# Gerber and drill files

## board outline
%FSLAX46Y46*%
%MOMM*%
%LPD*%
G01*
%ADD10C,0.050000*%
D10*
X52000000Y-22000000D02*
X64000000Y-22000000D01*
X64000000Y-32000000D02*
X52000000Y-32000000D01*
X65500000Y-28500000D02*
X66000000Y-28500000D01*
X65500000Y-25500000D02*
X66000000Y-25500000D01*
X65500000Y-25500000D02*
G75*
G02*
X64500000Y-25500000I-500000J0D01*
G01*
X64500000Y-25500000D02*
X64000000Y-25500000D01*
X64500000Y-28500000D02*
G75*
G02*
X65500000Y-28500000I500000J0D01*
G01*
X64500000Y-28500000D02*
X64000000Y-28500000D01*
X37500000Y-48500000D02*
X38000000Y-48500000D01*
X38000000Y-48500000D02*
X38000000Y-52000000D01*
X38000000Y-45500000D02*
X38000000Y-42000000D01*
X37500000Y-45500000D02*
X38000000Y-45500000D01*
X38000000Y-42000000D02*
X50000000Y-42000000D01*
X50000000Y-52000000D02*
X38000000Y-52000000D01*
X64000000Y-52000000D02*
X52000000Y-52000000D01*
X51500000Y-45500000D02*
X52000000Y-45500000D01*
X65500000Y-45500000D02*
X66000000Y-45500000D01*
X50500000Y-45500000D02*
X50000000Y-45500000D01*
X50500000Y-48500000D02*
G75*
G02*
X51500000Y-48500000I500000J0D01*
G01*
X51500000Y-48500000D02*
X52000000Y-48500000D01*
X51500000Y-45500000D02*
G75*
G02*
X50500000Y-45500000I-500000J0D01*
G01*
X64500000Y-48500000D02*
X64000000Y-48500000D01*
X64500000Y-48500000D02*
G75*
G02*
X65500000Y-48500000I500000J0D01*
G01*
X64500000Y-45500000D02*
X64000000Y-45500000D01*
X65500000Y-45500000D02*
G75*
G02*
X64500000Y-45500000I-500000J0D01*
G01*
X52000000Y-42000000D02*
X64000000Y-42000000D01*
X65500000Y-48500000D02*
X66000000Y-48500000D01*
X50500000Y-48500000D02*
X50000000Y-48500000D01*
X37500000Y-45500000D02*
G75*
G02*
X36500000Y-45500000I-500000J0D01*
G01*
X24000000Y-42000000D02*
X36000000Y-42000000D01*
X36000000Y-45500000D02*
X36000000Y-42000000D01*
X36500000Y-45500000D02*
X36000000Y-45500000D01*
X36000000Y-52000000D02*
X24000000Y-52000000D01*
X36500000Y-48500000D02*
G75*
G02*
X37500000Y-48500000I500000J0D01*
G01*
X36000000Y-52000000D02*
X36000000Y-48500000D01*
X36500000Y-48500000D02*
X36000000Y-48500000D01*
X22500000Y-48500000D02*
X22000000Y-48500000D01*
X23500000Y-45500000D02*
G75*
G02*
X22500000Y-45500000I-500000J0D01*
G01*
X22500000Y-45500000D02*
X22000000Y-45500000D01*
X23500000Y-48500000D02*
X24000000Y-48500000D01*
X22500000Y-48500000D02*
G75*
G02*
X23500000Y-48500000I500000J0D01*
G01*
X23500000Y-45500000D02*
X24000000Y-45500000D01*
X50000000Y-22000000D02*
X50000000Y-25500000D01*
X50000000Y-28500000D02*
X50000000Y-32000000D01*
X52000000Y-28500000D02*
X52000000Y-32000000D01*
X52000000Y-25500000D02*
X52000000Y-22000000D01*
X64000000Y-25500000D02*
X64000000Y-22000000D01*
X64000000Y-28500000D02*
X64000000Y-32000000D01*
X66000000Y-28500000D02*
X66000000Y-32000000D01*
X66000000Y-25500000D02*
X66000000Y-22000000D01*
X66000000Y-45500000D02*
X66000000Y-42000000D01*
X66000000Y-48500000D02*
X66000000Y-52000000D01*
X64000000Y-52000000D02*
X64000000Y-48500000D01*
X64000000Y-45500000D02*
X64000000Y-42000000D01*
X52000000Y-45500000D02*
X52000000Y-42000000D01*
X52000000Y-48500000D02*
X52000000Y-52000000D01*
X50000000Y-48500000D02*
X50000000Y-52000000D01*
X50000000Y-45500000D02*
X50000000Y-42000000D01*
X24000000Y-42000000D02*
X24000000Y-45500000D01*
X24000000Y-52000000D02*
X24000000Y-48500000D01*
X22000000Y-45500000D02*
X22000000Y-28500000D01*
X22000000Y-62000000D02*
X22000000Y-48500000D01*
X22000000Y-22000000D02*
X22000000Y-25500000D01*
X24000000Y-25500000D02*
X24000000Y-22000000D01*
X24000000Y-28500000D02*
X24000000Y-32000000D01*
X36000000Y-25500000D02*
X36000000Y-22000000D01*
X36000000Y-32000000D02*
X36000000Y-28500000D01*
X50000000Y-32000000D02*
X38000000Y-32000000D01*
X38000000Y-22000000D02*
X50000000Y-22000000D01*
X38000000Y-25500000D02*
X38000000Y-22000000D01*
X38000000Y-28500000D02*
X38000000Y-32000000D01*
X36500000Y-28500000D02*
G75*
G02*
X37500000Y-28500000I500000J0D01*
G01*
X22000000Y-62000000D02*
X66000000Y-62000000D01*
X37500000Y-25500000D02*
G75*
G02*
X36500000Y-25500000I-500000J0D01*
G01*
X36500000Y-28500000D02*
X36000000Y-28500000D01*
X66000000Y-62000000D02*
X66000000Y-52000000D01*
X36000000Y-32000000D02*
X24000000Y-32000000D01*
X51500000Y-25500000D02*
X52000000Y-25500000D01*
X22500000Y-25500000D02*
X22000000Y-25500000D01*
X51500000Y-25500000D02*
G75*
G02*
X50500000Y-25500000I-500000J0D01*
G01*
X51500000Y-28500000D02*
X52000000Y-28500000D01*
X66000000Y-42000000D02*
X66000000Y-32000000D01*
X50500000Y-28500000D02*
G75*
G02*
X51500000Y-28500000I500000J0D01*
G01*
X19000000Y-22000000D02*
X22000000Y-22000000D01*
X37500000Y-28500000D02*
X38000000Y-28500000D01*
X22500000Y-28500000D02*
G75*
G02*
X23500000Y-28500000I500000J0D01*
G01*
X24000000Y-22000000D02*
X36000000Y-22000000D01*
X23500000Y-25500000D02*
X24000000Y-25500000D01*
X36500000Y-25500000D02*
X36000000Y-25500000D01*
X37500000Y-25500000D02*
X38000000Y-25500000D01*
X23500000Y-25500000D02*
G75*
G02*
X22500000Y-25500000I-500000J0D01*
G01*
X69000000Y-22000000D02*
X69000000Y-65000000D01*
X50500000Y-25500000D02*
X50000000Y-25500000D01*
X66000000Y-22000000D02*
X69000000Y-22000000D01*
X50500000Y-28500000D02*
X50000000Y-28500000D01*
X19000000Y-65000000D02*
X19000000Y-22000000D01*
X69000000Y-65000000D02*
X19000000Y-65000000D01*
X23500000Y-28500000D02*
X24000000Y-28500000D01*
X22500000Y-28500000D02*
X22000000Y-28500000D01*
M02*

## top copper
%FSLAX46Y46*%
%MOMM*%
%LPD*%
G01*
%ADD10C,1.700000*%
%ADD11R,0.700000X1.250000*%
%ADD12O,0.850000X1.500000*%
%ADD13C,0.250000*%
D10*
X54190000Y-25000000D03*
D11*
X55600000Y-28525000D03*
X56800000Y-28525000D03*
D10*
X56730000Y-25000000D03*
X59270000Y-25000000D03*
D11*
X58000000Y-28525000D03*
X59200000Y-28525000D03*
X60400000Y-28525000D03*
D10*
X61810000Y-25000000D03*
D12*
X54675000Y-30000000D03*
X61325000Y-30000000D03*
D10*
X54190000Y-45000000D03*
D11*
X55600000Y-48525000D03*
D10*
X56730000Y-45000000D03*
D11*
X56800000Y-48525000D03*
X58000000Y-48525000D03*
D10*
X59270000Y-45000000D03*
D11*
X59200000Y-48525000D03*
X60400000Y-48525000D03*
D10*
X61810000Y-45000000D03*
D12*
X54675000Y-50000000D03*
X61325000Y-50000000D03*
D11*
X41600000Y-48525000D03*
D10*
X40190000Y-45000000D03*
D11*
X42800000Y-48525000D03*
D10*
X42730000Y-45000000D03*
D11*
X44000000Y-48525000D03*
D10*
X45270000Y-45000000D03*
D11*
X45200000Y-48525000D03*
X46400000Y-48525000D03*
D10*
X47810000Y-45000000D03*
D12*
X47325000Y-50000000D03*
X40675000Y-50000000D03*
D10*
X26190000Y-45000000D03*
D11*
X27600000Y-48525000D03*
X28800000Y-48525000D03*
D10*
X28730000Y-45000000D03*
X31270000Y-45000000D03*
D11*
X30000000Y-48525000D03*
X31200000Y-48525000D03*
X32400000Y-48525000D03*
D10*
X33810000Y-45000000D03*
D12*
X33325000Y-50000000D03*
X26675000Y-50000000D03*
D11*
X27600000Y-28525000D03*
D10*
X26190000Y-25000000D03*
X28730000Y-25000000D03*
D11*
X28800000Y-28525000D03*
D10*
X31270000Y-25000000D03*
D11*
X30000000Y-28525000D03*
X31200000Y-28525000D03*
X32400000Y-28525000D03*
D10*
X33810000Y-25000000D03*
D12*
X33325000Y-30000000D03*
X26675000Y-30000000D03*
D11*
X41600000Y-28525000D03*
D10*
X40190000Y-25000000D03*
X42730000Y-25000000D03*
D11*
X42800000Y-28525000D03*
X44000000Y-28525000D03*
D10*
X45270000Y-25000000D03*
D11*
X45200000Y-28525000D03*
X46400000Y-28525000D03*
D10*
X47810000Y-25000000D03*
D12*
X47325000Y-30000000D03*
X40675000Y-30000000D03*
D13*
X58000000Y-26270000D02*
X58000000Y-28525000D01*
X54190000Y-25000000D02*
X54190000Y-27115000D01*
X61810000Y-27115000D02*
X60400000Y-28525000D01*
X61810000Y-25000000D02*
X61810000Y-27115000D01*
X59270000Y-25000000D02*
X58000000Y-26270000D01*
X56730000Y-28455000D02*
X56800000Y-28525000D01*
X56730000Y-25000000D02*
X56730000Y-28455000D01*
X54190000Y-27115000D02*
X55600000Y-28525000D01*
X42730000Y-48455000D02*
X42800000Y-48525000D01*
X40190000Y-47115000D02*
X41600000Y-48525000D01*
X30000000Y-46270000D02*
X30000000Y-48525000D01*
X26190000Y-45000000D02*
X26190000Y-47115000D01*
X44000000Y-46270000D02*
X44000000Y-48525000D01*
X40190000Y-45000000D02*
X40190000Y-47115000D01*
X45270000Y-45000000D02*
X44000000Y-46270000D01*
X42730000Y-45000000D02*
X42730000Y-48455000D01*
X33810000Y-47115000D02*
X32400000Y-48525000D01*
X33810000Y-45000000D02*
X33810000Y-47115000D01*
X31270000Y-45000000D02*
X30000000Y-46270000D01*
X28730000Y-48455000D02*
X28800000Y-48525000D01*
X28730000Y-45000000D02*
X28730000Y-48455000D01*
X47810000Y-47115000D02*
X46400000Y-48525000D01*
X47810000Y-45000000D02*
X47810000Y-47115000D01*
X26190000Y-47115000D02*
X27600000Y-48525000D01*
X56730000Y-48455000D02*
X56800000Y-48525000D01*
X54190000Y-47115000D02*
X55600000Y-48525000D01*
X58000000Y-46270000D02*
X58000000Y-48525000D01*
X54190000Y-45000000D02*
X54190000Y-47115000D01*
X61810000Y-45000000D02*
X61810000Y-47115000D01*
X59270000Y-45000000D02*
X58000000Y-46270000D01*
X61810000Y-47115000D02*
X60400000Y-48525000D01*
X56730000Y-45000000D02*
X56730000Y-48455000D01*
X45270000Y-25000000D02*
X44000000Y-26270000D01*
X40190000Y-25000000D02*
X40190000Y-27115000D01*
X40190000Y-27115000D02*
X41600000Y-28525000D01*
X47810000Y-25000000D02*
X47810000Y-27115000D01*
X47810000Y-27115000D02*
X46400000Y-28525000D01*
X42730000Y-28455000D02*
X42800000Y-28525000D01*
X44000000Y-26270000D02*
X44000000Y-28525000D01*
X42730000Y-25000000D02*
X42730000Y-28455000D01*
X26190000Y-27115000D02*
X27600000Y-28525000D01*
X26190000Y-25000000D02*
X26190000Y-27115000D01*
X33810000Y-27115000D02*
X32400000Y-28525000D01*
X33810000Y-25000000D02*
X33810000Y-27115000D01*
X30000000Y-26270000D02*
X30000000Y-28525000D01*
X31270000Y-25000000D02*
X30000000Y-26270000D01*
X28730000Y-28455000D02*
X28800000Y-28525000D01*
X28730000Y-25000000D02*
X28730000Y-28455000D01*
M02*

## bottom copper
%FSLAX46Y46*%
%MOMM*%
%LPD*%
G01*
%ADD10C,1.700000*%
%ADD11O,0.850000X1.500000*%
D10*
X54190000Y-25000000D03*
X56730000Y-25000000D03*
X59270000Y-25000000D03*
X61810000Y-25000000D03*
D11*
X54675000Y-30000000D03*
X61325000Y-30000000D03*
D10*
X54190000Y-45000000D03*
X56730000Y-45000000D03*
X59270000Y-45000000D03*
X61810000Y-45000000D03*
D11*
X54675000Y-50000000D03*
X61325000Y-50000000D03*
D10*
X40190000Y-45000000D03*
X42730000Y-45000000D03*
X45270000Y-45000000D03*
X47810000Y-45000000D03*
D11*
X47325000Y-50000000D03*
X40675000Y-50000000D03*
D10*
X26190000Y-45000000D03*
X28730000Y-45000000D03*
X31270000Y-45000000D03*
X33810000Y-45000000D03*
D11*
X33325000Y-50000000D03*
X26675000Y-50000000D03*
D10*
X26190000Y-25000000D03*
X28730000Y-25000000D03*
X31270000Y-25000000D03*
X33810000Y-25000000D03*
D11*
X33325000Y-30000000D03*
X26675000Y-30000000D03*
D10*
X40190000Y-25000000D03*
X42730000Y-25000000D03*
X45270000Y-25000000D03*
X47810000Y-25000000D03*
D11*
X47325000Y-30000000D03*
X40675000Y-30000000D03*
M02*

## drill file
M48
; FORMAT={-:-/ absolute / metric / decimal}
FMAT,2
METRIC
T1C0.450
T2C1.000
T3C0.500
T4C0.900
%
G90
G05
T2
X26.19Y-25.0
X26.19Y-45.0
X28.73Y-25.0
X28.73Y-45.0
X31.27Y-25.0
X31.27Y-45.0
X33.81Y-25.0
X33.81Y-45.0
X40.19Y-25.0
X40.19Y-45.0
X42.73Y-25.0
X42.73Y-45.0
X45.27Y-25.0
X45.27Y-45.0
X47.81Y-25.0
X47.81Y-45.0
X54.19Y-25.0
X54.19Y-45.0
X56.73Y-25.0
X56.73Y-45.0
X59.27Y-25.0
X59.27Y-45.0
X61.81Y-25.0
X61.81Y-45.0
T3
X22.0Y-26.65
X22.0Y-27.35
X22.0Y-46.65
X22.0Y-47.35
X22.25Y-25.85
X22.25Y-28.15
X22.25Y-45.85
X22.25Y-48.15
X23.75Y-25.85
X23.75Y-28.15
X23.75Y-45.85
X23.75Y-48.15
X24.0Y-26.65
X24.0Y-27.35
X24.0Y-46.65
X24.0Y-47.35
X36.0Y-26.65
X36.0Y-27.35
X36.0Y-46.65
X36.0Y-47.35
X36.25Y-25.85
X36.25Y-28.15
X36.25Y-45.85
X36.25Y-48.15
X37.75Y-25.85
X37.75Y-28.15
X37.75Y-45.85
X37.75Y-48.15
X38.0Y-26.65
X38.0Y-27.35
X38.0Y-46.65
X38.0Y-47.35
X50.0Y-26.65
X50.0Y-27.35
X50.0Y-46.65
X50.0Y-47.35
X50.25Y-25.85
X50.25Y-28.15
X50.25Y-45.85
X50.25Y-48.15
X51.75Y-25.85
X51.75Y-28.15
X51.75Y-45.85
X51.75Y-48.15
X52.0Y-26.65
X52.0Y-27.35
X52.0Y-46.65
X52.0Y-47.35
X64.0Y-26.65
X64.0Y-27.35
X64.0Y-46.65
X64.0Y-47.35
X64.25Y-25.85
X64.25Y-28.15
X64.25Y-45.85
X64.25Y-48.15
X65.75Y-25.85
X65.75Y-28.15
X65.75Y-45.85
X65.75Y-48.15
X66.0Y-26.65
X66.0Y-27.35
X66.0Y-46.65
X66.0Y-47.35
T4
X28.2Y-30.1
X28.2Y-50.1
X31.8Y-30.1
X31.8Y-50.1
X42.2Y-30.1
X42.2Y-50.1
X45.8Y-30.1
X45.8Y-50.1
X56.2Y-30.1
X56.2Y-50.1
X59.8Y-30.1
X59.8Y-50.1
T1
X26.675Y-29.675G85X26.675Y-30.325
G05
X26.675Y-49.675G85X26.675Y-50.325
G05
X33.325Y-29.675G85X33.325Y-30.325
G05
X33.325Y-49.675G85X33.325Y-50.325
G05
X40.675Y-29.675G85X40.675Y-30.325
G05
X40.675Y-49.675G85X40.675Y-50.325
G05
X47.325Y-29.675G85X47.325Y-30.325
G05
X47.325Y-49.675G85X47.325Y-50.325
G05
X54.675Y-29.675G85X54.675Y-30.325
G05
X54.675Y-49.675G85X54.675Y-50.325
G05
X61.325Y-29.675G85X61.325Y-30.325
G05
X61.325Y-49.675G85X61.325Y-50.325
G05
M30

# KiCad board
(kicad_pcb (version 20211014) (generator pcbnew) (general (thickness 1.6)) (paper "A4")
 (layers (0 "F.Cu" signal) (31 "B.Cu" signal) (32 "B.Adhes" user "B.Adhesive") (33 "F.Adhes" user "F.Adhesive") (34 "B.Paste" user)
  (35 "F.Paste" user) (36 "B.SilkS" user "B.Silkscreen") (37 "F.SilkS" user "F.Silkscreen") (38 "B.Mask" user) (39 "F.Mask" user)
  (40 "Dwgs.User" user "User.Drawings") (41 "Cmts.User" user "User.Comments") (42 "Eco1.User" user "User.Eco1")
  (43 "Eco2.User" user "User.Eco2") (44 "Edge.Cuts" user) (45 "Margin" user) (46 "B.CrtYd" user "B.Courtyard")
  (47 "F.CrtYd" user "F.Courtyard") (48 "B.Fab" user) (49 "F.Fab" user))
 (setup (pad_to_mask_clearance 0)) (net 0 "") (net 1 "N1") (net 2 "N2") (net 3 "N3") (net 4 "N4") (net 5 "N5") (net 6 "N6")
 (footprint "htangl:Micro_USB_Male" (layer "F.Cu") (at 58 30)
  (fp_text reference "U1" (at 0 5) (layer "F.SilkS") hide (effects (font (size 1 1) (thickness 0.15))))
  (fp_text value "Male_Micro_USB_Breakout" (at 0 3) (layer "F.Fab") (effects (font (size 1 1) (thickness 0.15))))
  (pad "" np_thru_hole circle (at 1.8 0.1) (size 0.9 0.9) (drill 0.9) (layers *.Cu *.Mask))
  (pad "" np_thru_hole circle (at -1.8 0.1) (size 0.9 0.9) (drill 0.9) (layers *.Cu *.Mask))
  (pad "1" thru_hole circle (at -3.81 -5) (size 1.7 1.7) (drill 1) (layers *.Cu *.Mask))
  (pad "1" smd rect (at -2.4 -1.475) (size 0.7 1.25) (layers "F.Cu" "F.Paste" "F.Mask"))
  (pad "2" smd rect (at -1.2 -1.475) (size 0.7 1.25) (layers "F.Cu" "F.Paste" "F.Mask"))
  (pad "2" thru_hole circle (at -1.27 -5) (size 1.7 1.7) (drill 1) (layers *.Cu *.Mask))
  (pad "3" thru_hole circle (at 1.27 -5) (size 1.7 1.7) (drill 1) (layers *.Cu *.Mask))
  (pad "3" smd rect (at 0 -1.475) (size 0.7 1.25) (layers "F.Cu" "F.Paste" "F.Mask"))
  (pad "4" smd rect (at 1.2 -1.475) (size 0.7 1.25) (layers "F.Cu" "F.Paste" "F.Mask"))
  (pad "5" smd rect (at 2.4 -1.475) (size 0.7 1.25) (layers "F.Cu" "F.Paste" "F.Mask"))
  (pad "5" thru_hole circle (at 3.81 -5) (size 1.7 1.7) (drill 1) (layers *.Cu *.Mask))
  (pad "6" thru_hole oval (at -3.325 0) (size 0.85 1.5) (drill oval 0.45 1.1) (layers *.Cu *.Mask))
  (pad "6" thru_hole oval (at 3.325 0) (size 0.85 1.5) (drill oval 0.45 1.1) (layers *.Cu *.Mask)))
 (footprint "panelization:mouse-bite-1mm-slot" (layer "F.Cu") (at 65 27 90)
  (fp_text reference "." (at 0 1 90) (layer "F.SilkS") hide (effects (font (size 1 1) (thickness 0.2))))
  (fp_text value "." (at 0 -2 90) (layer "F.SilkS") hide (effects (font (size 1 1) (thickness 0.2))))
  (pad "" np_thru_hole circle locked (at 0.35 -1 90) (size 0.5 0.5) (drill 0.5) (layers *.Cu *.Mask))
  (pad "" np_thru_hole circle locked (at -1.15 0.75 90) (size 0.5 0.5) (drill 0.5) (layers *.Cu *.Mask))
  (pad "" np_thru_hole circle locked (at 0.35 1 90) (size 0.5 0.5) (drill 0.5) (layers *.Cu *.Mask))
  (pad "" np_thru_hole circle locked (at 1.15 0.75 90) (size 0.5 0.5) (drill 0.5) (layers *.Cu *.Mask))
  (pad "" np_thru_hole circle locked (at 1.15 -0.75 90) (size 0.5 0.5) (drill 0.5) (layers *.Cu *.Mask))
  (pad "" np_thru_hole circle locked (at -0.35 1 90) (size 0.5 0.5) (drill 0.5) (layers *.Cu *.Mask))
  (pad "" np_thru_hole circle locked (at -1.15 -0.75 90) (size 0.5 0.5) (drill 0.5) (layers *.Cu *.Mask))
  (pad "" np_thru_hole circle locked (at -0.35 -1 90) (size 0.5 0.5) (drill 0.5) (layers *.Cu *.Mask)))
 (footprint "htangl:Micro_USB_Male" (layer "F.Cu") (at 58 50)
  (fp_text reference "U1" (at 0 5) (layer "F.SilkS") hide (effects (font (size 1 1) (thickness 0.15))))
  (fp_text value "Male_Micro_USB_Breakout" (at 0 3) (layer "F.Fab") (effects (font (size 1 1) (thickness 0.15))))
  (pad "" np_thru_hole circle (at 1.8 0.1) (size 0.9 0.9) (drill 0.9) (layers *.Cu *.Mask))
  (pad "" np_thru_hole circle (at -1.8 0.1) (size 0.9 0.9) (drill 0.9) (layers *.Cu *.Mask))
  (pad "1" thru_hole circle (at -3.81 -5) (size 1.7 1.7) (drill 1) (layers *.Cu *.Mask))
  (pad "1" smd rect (at -2.4 -1.475) (size 0.7 1.25) (layers "F.Cu" "F.Paste" "F.Mask"))
  (pad "2" thru_hole circle (at -1.27 -5) (size 1.7 1.7) (drill 1) (layers *.Cu *.Mask))
  (pad "2" smd rect (at -1.2 -1.475) (size 0.7 1.25) (layers "F.Cu" "F.Paste" "F.Mask"))
  (pad "3" smd rect (at 0 -1.475) (size 0.7 1.25) (layers "F.Cu" "F.Paste" "F.Mask"))
  (pad "3" thru_hole circle (at 1.27 -5) (size 1.7 1.7) (drill 1) (layers *.Cu *.Mask))
  (pad "4" smd rect (at 1.2 -1.475) (size 0.7 1.25) (layers "F.Cu" "F.Paste" "F.Mask"))
  (pad "5" smd rect (at 2.4 -1.475) (size 0.7 1.25) (layers "F.Cu" "F.Paste" "F.Mask"))
  (pad "5" thru_hole circle (at 3.81 -5) (size 1.7 1.7) (drill 1) (layers *.Cu *.Mask))
  (pad "6" thru_hole oval (at -3.325 0) (size 0.85 1.5) (drill oval 0.45 1.1) (layers *.Cu *.Mask))
  (pad "6" thru_hole oval (at 3.325 0) (size 0.85 1.5) (drill oval 0.45 1.1) (layers *.Cu *.Mask)))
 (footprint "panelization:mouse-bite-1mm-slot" (layer "F.Cu") (at 51 47 90)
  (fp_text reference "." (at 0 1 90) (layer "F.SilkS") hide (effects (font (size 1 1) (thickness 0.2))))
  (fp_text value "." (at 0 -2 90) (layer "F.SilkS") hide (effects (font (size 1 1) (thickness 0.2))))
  (pad "" np_thru_hole circle locked (at -1.15 -0.75 90) (size 0.5 0.5) (drill 0.5) (layers *.Cu *.Mask))
  (pad "" np_thru_hole circle locked (at -0.35 1 90) (size 0.5 0.5) (drill 0.5) (layers *.Cu *.Mask))
  (pad "" np_thru_hole circle locked (at -0.35 -1 90) (size 0.5 0.5) (drill 0.5) (layers *.Cu *.Mask))
  (pad "" np_thru_hole circle locked (at 0.35 -1 90) (size 0.5 0.5) (drill 0.5) (layers *.Cu *.Mask))
  (pad "" np_thru_hole circle locked (at 1.15 -0.75 90) (size 0.5 0.5) (drill 0.5) (layers *.Cu *.Mask))
  (pad "" np_thru_hole circle locked (at 1.15 0.75 90) (size 0.5 0.5) (drill 0.5) (layers *.Cu *.Mask))
  (pad "" np_thru_hole circle locked (at -1.15 0.75 90) (size 0.5 0.5) (drill 0.5) (layers *.Cu *.Mask))
  (pad "" np_thru_hole circle locked (at 0.35 1 90) (size 0.5 0.5) (drill 0.5) (layers *.Cu *.Mask)))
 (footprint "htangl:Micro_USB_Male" (layer "F.Cu") (at 44 50)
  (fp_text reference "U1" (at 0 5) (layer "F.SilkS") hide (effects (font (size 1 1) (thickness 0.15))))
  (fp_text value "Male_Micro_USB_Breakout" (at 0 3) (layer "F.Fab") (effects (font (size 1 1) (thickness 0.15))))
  (pad "" np_thru_hole circle (at -1.8 0.1) (size 0.9 0.9) (drill 0.9) (layers *.Cu *.Mask))
  (pad "" np_thru_hole circle (at 1.8 0.1) (size 0.9 0.9) (drill 0.9) (layers *.Cu *.Mask))
  (pad "1" smd rect (at -2.4 -1.475) (size 0.7 1.25) (layers "F.Cu" "F.Paste" "F.Mask"))
  (pad "1" thru_hole circle (at -3.81 -5) (size 1.7 1.7) (drill 1) (layers *.Cu *.Mask))
  (pad "2" smd rect (at -1.2 -1.475) (size 0.7 1.25) (layers "F.Cu" "F.Paste" "F.Mask"))
  (pad "2" thru_hole circle (at -1.27 -5) (size 1.7 1.7) (drill 1) (layers *.Cu *.Mask))
  (pad "3" smd rect (at 0 -1.475) (size 0.7 1.25) (layers "F.Cu" "F.Paste" "F.Mask"))
  (pad "3" thru_hole circle (at 1.27 -5) (size 1.7 1.7) (drill 1) (layers *.Cu *.Mask))
  (pad "4" smd rect (at 1.2 -1.475) (size 0.7 1.25) (layers "F.Cu" "F.Paste" "F.Mask"))
  (pad "5" smd rect (at 2.4 -1.475) (size 0.7 1.25) (layers "F.Cu" "F.Paste" "F.Mask"))
  (pad "5" thru_hole circle (at 3.81 -5) (size 1.7 1.7) (drill 1) (layers *.Cu *.Mask))
  (pad "6" thru_hole oval (at 3.325 0) (size 0.85 1.5) (drill oval 0.45 1.1) (layers *.Cu *.Mask))
  (pad "6" thru_hole oval (at -3.325 0) (size 0.85 1.5) (drill oval 0.45 1.1) (layers *.Cu *.Mask)))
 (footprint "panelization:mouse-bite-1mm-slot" (layer "F.Cu") (at 65 47 90)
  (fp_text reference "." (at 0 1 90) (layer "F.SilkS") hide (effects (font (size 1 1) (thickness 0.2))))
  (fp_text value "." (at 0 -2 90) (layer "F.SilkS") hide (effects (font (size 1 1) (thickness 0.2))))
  (pad "" np_thru_hole circle locked (at 0.35 1 90) (size 0.5 0.5) (drill 0.5) (layers *.Cu *.Mask))
  (pad "" np_thru_hole circle locked (at 1.15 -0.75 90) (size 0.5 0.5) (drill 0.5) (layers *.Cu *.Mask))
  (pad "" np_thru_hole circle locked (at 0.35 -1 90) (size 0.5 0.5) (drill 0.5) (layers *.Cu *.Mask))
  (pad "" np_thru_hole circle locked (at -0.35 -1 90) (size 0.5 0.5) (drill 0.5) (layers *.Cu *.Mask))
  (pad "" np_thru_hole circle locked (at -1.15 -0.75 90) (size 0.5 0.5) (drill 0.5) (layers *.Cu *.Mask))
  (pad "" np_thru_hole circle locked (at -0.35 1 90) (size 0.5 0.5) (drill 0.5) (layers *.Cu *.Mask))
  (pad "" np_thru_hole circle locked (at 1.15 0.75 90) (size 0.5 0.5) (drill 0.5) (layers *.Cu *.Mask))
  (pad "" np_thru_hole circle locked (at -1.15 0.75 90) (size 0.5 0.5) (drill 0.5) (layers *.Cu *.Mask)))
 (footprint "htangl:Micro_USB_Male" (layer "F.Cu") (at 30 50)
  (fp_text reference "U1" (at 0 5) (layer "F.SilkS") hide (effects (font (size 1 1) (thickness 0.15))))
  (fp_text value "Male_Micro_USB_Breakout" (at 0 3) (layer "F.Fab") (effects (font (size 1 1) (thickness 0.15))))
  (pad "" np_thru_hole circle (at 1.8 0.1) (size 0.9 0.9) (drill 0.9) (layers *.Cu *.Mask))
  (pad "" np_thru_hole circle (at -1.8 0.1) (size 0.9 0.9) (drill 0.9) (layers *.Cu *.Mask))
  (pad "1" thru_hole circle (at -3.81 -5) (size 1.7 1.7) (drill 1) (layers *.Cu *.Mask))
  (pad "1" smd rect (at -2.4 -1.475) (size 0.7 1.25) (layers "F.Cu" "F.Paste" "F.Mask"))
  (pad "2" smd rect (at -1.2 -1.475) (size 0.7 1.25) (layers "F.Cu" "F.Paste" "F.Mask"))
  (pad "2" thru_hole circle (at -1.27 -5) (size 1.7 1.7) (drill 1) (layers *.Cu *.Mask))
  (pad "3" thru_hole circle (at 1.27 -5) (size 1.7 1.7) (drill 1) (layers *.Cu *.Mask))
  (pad "3" smd rect (at 0 -1.475) (size 0.7 1.25) (layers "F.Cu" "F.Paste" "F.Mask"))
  (pad "4" smd rect (at 1.2 -1.475) (size 0.7 1.25) (layers "F.Cu" "F.Paste" "F.Mask"))
  (pad "5" smd rect (at 2.4 -1.475) (size 0.7 1.25) (layers "F.Cu" "F.Paste" "F.Mask"))
  (pad "5" thru_hole circle (at 3.81 -5) (size 1.7 1.7) (drill 1) (layers *.Cu *.Mask))
  (pad "6" thru_hole oval (at 3.325 0) (size 0.85 1.5) (drill oval 0.45 1.1) (layers *.Cu *.Mask))
  (pad "6" thru_hole oval (at -3.325 0) (size 0.85 1.5) (drill oval 0.45 1.1) (layers *.Cu *.Mask)))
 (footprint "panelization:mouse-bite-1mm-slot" (layer "F.Cu") (at 37 47 90)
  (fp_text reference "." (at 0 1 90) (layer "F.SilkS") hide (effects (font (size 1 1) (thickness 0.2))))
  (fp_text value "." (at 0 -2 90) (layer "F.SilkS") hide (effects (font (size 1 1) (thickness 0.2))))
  (pad "" np_thru_hole circle locked (at -0.35 -1 90) (size 0.5 0.5) (drill 0.5) (layers *.Cu *.Mask))
  (pad "" np_thru_hole circle locked (at -0.35 1 90) (size 0.5 0.5) (drill 0.5) (layers *.Cu *.Mask))
  (pad "" np_thru_hole circle locked (at 1.15 -0.75 90) (size 0.5 0.5) (drill 0.5) (layers *.Cu *.Mask))
  (pad "" np_thru_hole circle locked (at -1.15 -0.75 90) (size 0.5 0.5) (drill 0.5) (layers *.Cu *.Mask))
  (pad "" np_thru_hole circle locked (at 1.15 0.75 90) (size 0.5 0.5) (drill 0.5) (layers *.Cu *.Mask))
  (pad "" np_thru_hole circle locked (at -1.15 0.75 90) (size 0.5 0.5) (drill 0.5) (layers *.Cu *.Mask))
  (pad "" np_thru_hole circle locked (at 0.35 -1 90) (size 0.5 0.5) (drill 0.5) (layers *.Cu *.Mask))
  (pad "" np_thru_hole circle locked (at 0.35 1 90) (size 0.5 0.5) (drill 0.5) (layers *.Cu *.Mask)))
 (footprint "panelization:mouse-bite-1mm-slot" (layer "F.Cu") (at 23 47 90)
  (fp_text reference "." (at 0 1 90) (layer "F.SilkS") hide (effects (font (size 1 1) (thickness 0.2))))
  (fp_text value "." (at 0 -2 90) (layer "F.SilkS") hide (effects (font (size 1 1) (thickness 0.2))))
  (pad "" np_thru_hole circle locked (at 0.35 1 90) (size 0.5 0.5) (drill 0.5) (layers *.Cu *.Mask))
  (pad "" np_thru_hole circle locked (at -0.35 -1 90) (size 0.5 0.5) (drill 0.5) (layers *.Cu *.Mask))
  (pad "" np_thru_hole circle locked (at 1.15 -0.75 90) (size 0.5 0.5) (drill 0.5) (layers *.Cu *.Mask))
  (pad "" np_thru_hole circle locked (at 1.15 0.75 90) (size 0.5 0.5) (drill 0.5) (layers *.Cu *.Mask))
  (pad "" np_thru_hole circle locked (at -1.15 0.75 90) (size 0.5 0.5) (drill 0.5) (layers *.Cu *.Mask))
  (pad "" np_thru_hole circle locked (at -1.15 -0.75 90) (size 0.5 0.5) (drill 0.5) (layers *.Cu *.Mask))
  (pad "" np_thru_hole circle locked (at 0.35 -1 90) (size 0.5 0.5) (drill 0.5) (layers *.Cu *.Mask))
  (pad "" np_thru_hole circle locked (at -0.35 1 90) (size 0.5 0.5) (drill 0.5) (layers *.Cu *.Mask)))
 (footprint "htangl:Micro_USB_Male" (layer "F.Cu") (at 30 30)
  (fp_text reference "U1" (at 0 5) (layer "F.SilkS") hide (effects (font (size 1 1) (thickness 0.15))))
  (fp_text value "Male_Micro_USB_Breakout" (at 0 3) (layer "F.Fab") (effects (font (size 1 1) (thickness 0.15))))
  (pad "" np_thru_hole circle (at 1.8 0.1) (size 0.9 0.9) (drill 0.9) (layers *.Cu *.Mask))
  (pad "" np_thru_hole circle (at -1.8 0.1) (size 0.9 0.9) (drill 0.9) (layers *.Cu *.Mask))
  (pad "1" smd rect (at -2.4 -1.475) (size 0.7 1.25) (layers "F.Cu" "F.Paste" "F.Mask") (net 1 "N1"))
  (pad "1" thru_hole circle (at -3.81 -5) (size 1.7 1.7) (drill 1) (layers *.Cu *.Mask) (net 1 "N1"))
  (pad "2" thru_hole circle (at -1.27 -5) (size 1.7 1.7) (drill 1) (layers *.Cu *.Mask) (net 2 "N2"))
  (pad "2" smd rect (at -1.2 -1.475) (size 0.7 1.25) (layers "F.Cu" "F.Paste" "F.Mask") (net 2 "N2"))
  (pad "3" thru_hole circle (at 1.27 -5) (size 1.7 1.7) (drill 1) (layers *.Cu *.Mask) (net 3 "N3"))
  (pad "3" smd rect (at 0 -1.475) (size 0.7 1.25) (layers "F.Cu" "F.Paste" "F.Mask") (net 3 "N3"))
  (pad "4" smd rect (at 1.2 -1.475) (size 0.7 1.25) (layers "F.Cu" "F.Paste" "F.Mask") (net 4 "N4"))
  (pad "5" smd rect (at 2.4 -1.475) (size 0.7 1.25) (layers "F.Cu" "F.Paste" "F.Mask") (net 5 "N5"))
  (pad "5" thru_hole circle (at 3.81 -5) (size 1.7 1.7) (drill 1) (layers *.Cu *.Mask) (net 5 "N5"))
  (pad "6" thru_hole oval (at 3.325 0) (size 0.85 1.5) (drill oval 0.45 1.1) (layers *.Cu *.Mask) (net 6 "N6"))
  (pad "6" thru_hole oval (at -3.325 0) (size 0.85 1.5) (drill oval 0.45 1.1) (layers *.Cu *.Mask) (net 6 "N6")))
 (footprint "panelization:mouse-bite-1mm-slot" (layer "F.Cu") (at 37 27 90)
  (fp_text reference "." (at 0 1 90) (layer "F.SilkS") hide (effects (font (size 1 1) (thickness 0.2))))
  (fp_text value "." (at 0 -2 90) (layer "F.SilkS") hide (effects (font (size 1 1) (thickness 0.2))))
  (pad "" np_thru_hole circle locked (at 1.15 -0.75 90) (size 0.5 0.5) (drill 0.5) (layers *.Cu *.Mask))
  (pad "" np_thru_hole circle locked (at -0.35 -1 90) (size 0.5 0.5) (drill 0.5) (layers *.Cu *.Mask))
  (pad "" np_thru_hole circle locked (at -0.35 1 90) (size 0.5 0.5) (drill 0.5) (layers *.Cu *.Mask))
  (pad "" np_thru_hole circle locked (at -1.15 -0.75 90) (size 0.5 0.5) (drill 0.5) (layers *.Cu *.Mask))
  (pad "" np_thru_hole circle locked (at 1.15 0.75 90) (size 0.5 0.5) (drill 0.5) (layers *.Cu *.Mask))
  (pad "" np_thru_hole circle locked (at 0.35 1 90) (size 0.5 0.5) (drill 0.5) (layers *.Cu *.Mask))
  (pad "" np_thru_hole circle locked (at -1.15 0.75 90) (size 0.5 0.5) (drill 0.5) (layers *.Cu *.Mask))
  (pad "" np_thru_hole circle locked (at 0.35 -1 90) (size 0.5 0.5) (drill 0.5) (layers *.Cu *.Mask)))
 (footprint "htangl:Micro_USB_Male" (layer "F.Cu") (at 44 30)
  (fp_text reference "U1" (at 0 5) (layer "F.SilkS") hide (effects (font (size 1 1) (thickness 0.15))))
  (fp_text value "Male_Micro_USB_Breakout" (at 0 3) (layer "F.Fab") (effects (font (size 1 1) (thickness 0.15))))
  (pad "" np_thru_hole circle (at -1.8 0.1) (size 0.9 0.9) (drill 0.9) (layers *.Cu *.Mask))
  (pad "" np_thru_hole circle (at 1.8 0.1) (size 0.9 0.9) (drill 0.9) (layers *.Cu *.Mask))
  (pad "1" smd rect (at -2.4 -1.475) (size 0.7 1.25) (layers "F.Cu" "F.Paste" "F.Mask"))
  (pad "1" thru_hole circle (at -3.81 -5) (size 1.7 1.7) (drill 1) (layers *.Cu *.Mask))
  (pad "2" thru_hole circle (at -1.27 -5) (size 1.7 1.7) (drill 1) (layers *.Cu *.Mask))
  (pad "2" smd rect (at -1.2 -1.475) (size 0.7 1.25) (layers "F.Cu" "F.Paste" "F.Mask"))
  (pad "3" smd rect (at 0 -1.475) (size 0.7 1.25) (layers "F.Cu" "F.Paste" "F.Mask"))
  (pad "3" thru_hole circle (at 1.27 -5) (size 1.7 1.7) (drill 1) (layers *.Cu *.Mask))
  (pad "4" smd rect (at 1.2 -1.475) (size 0.7 1.25) (layers "F.Cu" "F.Paste" "F.Mask"))
  (pad "5" smd rect (at 2.4 -1.475) (size 0.7 1.25) (layers "F.Cu" "F.Paste" "F.Mask"))
  (pad "5" thru_hole circle (at 3.81 -5) (size 1.7 1.7) (drill 1) (layers *.Cu *.Mask))
  (pad "6" thru_hole oval (at 3.325 0) (size 0.85 1.5) (drill oval 0.45 1.1) (layers *.Cu *.Mask))
  (pad "6" thru_hole oval (at -3.325 0) (size 0.85 1.5) (drill oval 0.45 1.1) (layers *.Cu *.Mask)))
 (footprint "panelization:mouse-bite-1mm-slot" (layer "F.Cu") (at 23 27 90)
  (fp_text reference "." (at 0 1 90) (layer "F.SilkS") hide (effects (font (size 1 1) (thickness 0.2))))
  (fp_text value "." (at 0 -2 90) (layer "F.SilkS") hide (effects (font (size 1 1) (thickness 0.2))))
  (pad "" np_thru_hole circle locked (at 0.35 -1 90) (size 0.5 0.5) (drill 0.5) (layers *.Cu *.Mask))
  (pad "" np_thru_hole circle locked (at -0.35 -1 90) (size 0.5 0.5) (drill 0.5) (layers *.Cu *.Mask))
  (pad "" np_thru_hole circle locked (at 0.35 1 90) (size 0.5 0.5) (drill 0.5) (layers *.Cu *.Mask))
  (pad "" np_thru_hole circle locked (at -0.35 1 90) (size 0.5 0.5) (drill 0.5) (layers *.Cu *.Mask))
  (pad "" np_thru_hole circle locked (at -1.15 0.75 90) (size 0.5 0.5) (drill 0.5) (layers *.Cu *.Mask))
  (pad "" np_thru_hole circle locked (at 1.15 -0.75 90) (size 0.5 0.5) (drill 0.5) (layers *.Cu *.Mask))
  (pad "" np_thru_hole circle locked (at -1.15 -0.75 90) (size 0.5 0.5) (drill 0.5) (layers *.Cu *.Mask))
  (pad "" np_thru_hole circle locked (at 1.15 0.75 90) (size 0.5 0.5) (drill 0.5) (layers *.Cu *.Mask)))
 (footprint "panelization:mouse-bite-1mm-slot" (layer "F.Cu") (at 51 27 90)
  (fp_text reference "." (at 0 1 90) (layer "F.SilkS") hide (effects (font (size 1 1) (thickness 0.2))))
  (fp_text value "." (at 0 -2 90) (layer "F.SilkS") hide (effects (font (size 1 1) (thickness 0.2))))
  (pad "" np_thru_hole circle locked (at 0.35 -1 90) (size 0.5 0.5) (drill 0.5) (layers *.Cu *.Mask))
  (pad "" np_thru_hole circle locked (at -0.35 1 90) (size 0.5 0.5) (drill 0.5) (layers *.Cu *.Mask))
  (pad "" np_thru_hole circle locked (at 1.15 0.75 90) (size 0.5 0.5) (drill 0.5) (layers *.Cu *.Mask))
  (pad "" np_thru_hole circle locked (at 1.15 -0.75 90) (size 0.5 0.5) (drill 0.5) (layers *.Cu *.Mask))
  (pad "" np_thru_hole circle locked (at -1.15 -0.75 90) (size 0.5 0.5) (drill 0.5) (layers *.Cu *.Mask))
  (pad "" np_thru_hole circle locked (at -0.35 -1 90) (size 0.5 0.5) (drill 0.5) (layers *.Cu *.Mask))
  (pad "" np_thru_hole circle locked (at -1.15 0.75 90) (size 0.5 0.5) (drill 0.5) (layers *.Cu *.Mask))
  (pad "" np_thru_hole circle locked (at 0.35 1 90) (size 0.5 0.5) (drill 0.5) (layers *.Cu *.Mask)))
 (gr_line (start 52 22) (end 64 22) (layer "Edge.Cuts") (width 0.05))
 (gr_line (start 64 32) (end 52 32) (layer "Edge.Cuts") (width 0.05))
 (gr_line (start 65.5 28.5) (end 66 28.5) (layer "Edge.Cuts") (width 0.05))
 (gr_line (start 65.5 25.5) (end 66 25.5) (layer "Edge.Cuts") (width 0.05))
 (gr_arc (start 65.5 25.5) (mid 65 26) (end 64.5 25.5) (layer "Edge.Cuts") (width 0.05))
 (gr_line (start 64.5 25.5) (end 64 25.5) (layer "Edge.Cuts") (width 0.05))
 (gr_arc (start 64.5 28.5) (mid 65 28) (end 65.5 28.5) (layer "Edge.Cuts") (width 0.05))
 (gr_line (start 64.5 28.5) (end 64 28.5) (layer "Edge.Cuts") (width 0.05))
 (gr_line (start 37.5 48.5) (end 38 48.5) (layer "Edge.Cuts") (width 0.05))
 (gr_line (start 38 48.5) (end 38 52) (layer "Edge.Cuts") (width 0.05))
 (gr_line (start 38 45.5) (end 38 42) (layer "Edge.Cuts") (width 0.05))
 (gr_line (start 37.5 45.5) (end 38 45.5) (layer "Edge.Cuts") (width 0.05))
 (gr_line (start 38 42) (end 50 42) (layer "Edge.Cuts") (width 0.05))
 (gr_line (start 50 52) (end 38 52) (layer "Edge.Cuts") (width 0.05))
 (gr_line (start 64 52) (end 52 52) (layer "Edge.Cuts") (width 0.05))
 (gr_line (start 51.5 45.5) (end 52 45.5) (layer "Edge.Cuts") (width 0.05))
 (gr_line (start 65.5 45.5) (end 66 45.5) (layer "Edge.Cuts") (width 0.05))
 (gr_line (start 50.5 45.5) (end 50 45.5) (layer "Edge.Cuts") (width 0.05))
 (gr_arc (start 50.5 48.5) (mid 51 48) (end 51.5 48.5) (layer "Edge.Cuts") (width 0.05))
 (gr_line (start 51.5 48.5) (end 52 48.5) (layer "Edge.Cuts") (width 0.05))
 (gr_arc (start 51.5 45.5) (mid 51 46) (end 50.5 45.5) (layer "Edge.Cuts") (width 0.05))
 (gr_line (start 64.5 48.5) (end 64 48.5) (layer "Edge.Cuts") (width 0.05))
 (gr_arc (start 64.5 48.5) (mid 65 48) (end 65.5 48.5) (layer "Edge.Cuts") (width 0.05))
 (gr_line (start 64.5 45.5) (end 64 45.5) (layer "Edge.Cuts") (width 0.05))
 (gr_arc (start 65.5 45.5) (mid 65 46) (end 64.5 45.5) (layer "Edge.Cuts") (width 0.05))
 (gr_line (start 52 42) (end 64 42) (layer "Edge.Cuts") (width 0.05))
 (gr_line (start 65.5 48.5) (end 66 48.5) (layer "Edge.Cuts") (width 0.05))
 (gr_line (start 50.5 48.5) (end 50 48.5) (layer "Edge.Cuts") (width 0.05))
 (gr_arc (start 37.5 45.5) (mid 37 46) (end 36.5 45.5) (layer "Edge.Cuts") (width 0.05))
 (gr_line (start 24 42) (end 36 42) (layer "Edge.Cuts") (width 0.05))
 (gr_line (start 36 45.5) (end 36 42) (layer "Edge.Cuts") (width 0.05))
 (gr_line (start 36.5 45.5) (end 36 45.5) (layer "Edge.Cuts") (width 0.05))
 (gr_line (start 36 52) (end 24 52) (layer "Edge.Cuts") (width 0.05))
 (gr_arc (start 36.5 48.5) (mid 37 48) (end 37.5 48.5) (layer "Edge.Cuts") (width 0.05))
 (gr_line (start 36 52) (end 36 48.5) (layer "Edge.Cuts") (width 0.05))
 (gr_line (start 36.5 48.5) (end 36 48.5) (layer "Edge.Cuts") (width 0.05))
 (gr_line (start 22.5 48.5) (end 22 48.5) (layer "Edge.Cuts") (width 0.05))
 (gr_arc (start 23.5 45.5) (mid 23 46) (end 22.5 45.5) (layer "Edge.Cuts") (width 0.05))
 (gr_line (start 22.5 45.5) (end 22 45.5) (layer "Edge.Cuts") (width 0.05))
 (gr_line (start 23.5 48.5) (end 24 48.5) (layer "Edge.Cuts") (width 0.05))
 (gr_arc (start 22.5 48.5) (mid 23 48) (end 23.5 48.5) (layer "Edge.Cuts") (width 0.05))
 (gr_line (start 23.5 45.5) (end 24 45.5) (layer "Edge.Cuts") (width 0.05))
 (gr_line (start 50 22) (end 50 25.5) (layer "Edge.Cuts") (width 0.05))
 (gr_line (start 50 28.5) (end 50 32) (layer "Edge.Cuts") (width 0.05))
 (gr_line (start 52 28.5) (end 52 32) (layer "Edge.Cuts") (width 0.05))
 (gr_line (start 52 25.5) (end 52 22) (layer "Edge.Cuts") (width 0.05))
 (gr_line (start 64 25.5) (end 64 22) (layer "Edge.Cuts") (width 0.05))
 (gr_line (start 64 28.5) (end 64 32) (layer "Edge.Cuts") (width 0.05))
 (gr_line (start 66 28.5) (end 66 32) (layer "Edge.Cuts") (width 0.05))
 (gr_line (start 66 25.5) (end 66 22) (layer "Edge.Cuts") (width 0.05))
 (gr_line (start 66 45.5) (end 66 42) (layer "Edge.Cuts") (width 0.05))
 (gr_line (start 66 48.5) (end 66 52) (layer "Edge.Cuts") (width 0.05))
 (gr_line (start 64 52) (end 64 48.5) (layer "Edge.Cuts") (width 0.05))
 (gr_line (start 64 45.5) (end 64 42) (layer "Edge.Cuts") (width 0.05))
 (gr_line (start 52 45.5) (end 52 42) (layer "Edge.Cuts") (width 0.05))
 (gr_line (start 52 48.5) (end 52 52) (layer "Edge.Cuts") (width 0.05))
 (gr_line (start 50 48.5) (end 50 52) (layer "Edge.Cuts") (width 0.05))
 (gr_line (start 50 45.5) (end 50 42) (layer "Edge.Cuts") (width 0.05))
 (gr_line (start 24 42) (end 24 45.5) (layer "Edge.Cuts") (width 0.05))
 (gr_line (start 24 52) (end 24 48.5) (layer "Edge.Cuts") (width 0.05))
 (gr_line (start 22 45.5) (end 22 28.5) (layer "Edge.Cuts") (width 0.05))
 (gr_line (start 22 62) (end 22 48.5) (layer "Edge.Cuts") (width 0.05))
 (gr_line (start 22 22) (end 22 25.5) (layer "Edge.Cuts") (width 0.05))
 (gr_line (start 24 25.5) (end 24 22) (layer "Edge.Cuts") (width 0.05))
 (gr_line (start 24 28.5) (end 24 32) (layer "Edge.Cuts") (width 0.05))
 (gr_line (start 36 25.5) (end 36 22) (layer "Edge.Cuts") (width 0.05))
 (gr_line (start 36 32) (end 36 28.5) (layer "Edge.Cuts") (width 0.05))
 (gr_line (start 50 32) (end 38 32) (layer "Edge.Cuts") (width 0.05))
 (gr_line (start 38 22) (end 50 22) (layer "Edge.Cuts") (width 0.05))
 (gr_line (start 38 25.5) (end 38 22) (layer "Edge.Cuts") (width 0.05))
 (gr_line (start 38 28.5) (end 38 32) (layer "Edge.Cuts") (width 0.05))
 (gr_arc (start 36.5 28.5) (mid 37 28) (end 37.5 28.5) (layer "Edge.Cuts") (width 0.05))
 (gr_line (start 22 62) (end 66 62) (layer "Edge.Cuts") (width 0.05))
 (gr_arc (start 37.5 25.5) (mid 37 26) (end 36.5 25.5) (layer "Edge.Cuts") (width 0.05))
 (gr_line (start 36.5 28.5) (end 36 28.5) (layer "Edge.Cuts") (width 0.05))
 (gr_line (start 66 62) (end 66 52) (layer "Edge.Cuts") (width 0.05))
 (gr_line (start 36 32) (end 24 32) (layer "Edge.Cuts") (width 0.05))
 (gr_line (start 51.5 25.5) (end 52 25.5) (layer "Edge.Cuts") (width 0.05))
 (gr_line (start 22.5 25.5) (end 22 25.5) (layer "Edge.Cuts") (width 0.05))
 (gr_arc (start 51.5 25.5) (mid 51 26) (end 50.5 25.5) (layer "Edge.Cuts") (width 0.05))
 (gr_line (start 51.5 28.5) (end 52 28.5) (layer "Edge.Cuts") (width 0.05))
 (gr_line (start 66 42) (end 66 32) (layer "Edge.Cuts") (width 0.05))
 (gr_arc (start 50.5 28.5) (mid 51 28) (end 51.5 28.5) (layer "Edge.Cuts") (width 0.05))
 (gr_line (start 19 22) (end 22 22) (layer "Edge.Cuts") (width 0.05))
 (gr_line (start 37.5 28.5) (end 38 28.5) (layer "Edge.Cuts") (width 0.05))
 (gr_arc (start 22.5 28.5) (mid 23 28) (end 23.5 28.5) (layer "Edge.Cuts") (width 0.05))
 (gr_line (start 24 22) (end 36 22) (layer "Edge.Cuts") (width 0.05))
 (gr_line (start 23.5 25.5) (end 24 25.5) (layer "Edge.Cuts") (width 0.05))
 (gr_line (start 36.5 25.5) (end 36 25.5) (layer "Edge.Cuts") (width 0.05))
 (gr_line (start 37.5 25.5) (end 38 25.5) (layer "Edge.Cuts") (width 0.05))
 (gr_arc (start 23.5 25.5) (mid 23 26) (end 22.5 25.5) (layer "Edge.Cuts") (width 0.05))
 (gr_line (start 69 22) (end 69 65) (layer "Edge.Cuts") (width 0.05))
 (gr_line (start 50.5 25.5) (end 50 25.5) (layer "Edge.Cuts") (width 0.05))
 (gr_line (start 66 22) (end 69 22) (layer "Edge.Cuts") (width 0.05))
 (gr_line (start 50.5 28.5) (end 50 28.5) (layer "Edge.Cuts") (width 0.05))
 (gr_line (start 19 65) (end 19 22) (layer "Edge.Cuts") (width 0.05))
 (gr_line (start 69 65) (end 19 65) (layer "Edge.Cuts") (width 0.05))
 (gr_line (start 23.5 28.5) (end 24 28.5) (layer "Edge.Cuts") (width 0.05))
 (gr_line (start 22.5 28.5) (end 22 28.5) (layer "Edge.Cuts") (width 0.05))
 (segment (start 58 26.27) (end 58 28.525) (width 0.25) (layer "F.Cu") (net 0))
 (segment (start 54.19 25) (end 54.19 27.115) (width 0.25) (layer "F.Cu") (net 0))
 (segment (start 61.81 27.115) (end 60.4 28.525) (width 0.25) (layer "F.Cu") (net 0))
 (segment (start 61.81 25) (end 61.81 27.115) (width 0.25) (layer "F.Cu") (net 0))
 (segment (start 59.27 25) (end 58 26.27) (width 0.25) (layer "F.Cu") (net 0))
 (segment (start 56.73 28.455) (end 56.8 28.525) (width 0.25) (layer "F.Cu") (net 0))
 (segment (start 56.73 25) (end 56.73 28.455) (width 0.25) (layer "F.Cu") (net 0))
 (segment (start 54.19 27.115) (end 55.6 28.525) (width 0.25) (layer "F.Cu") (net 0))
 (segment (start 42.73 48.455) (end 42.8 48.525) (width 0.25) (layer "F.Cu") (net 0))
 (segment (start 40.19 47.115) (end 41.6 48.525) (width 0.25) (layer "F.Cu") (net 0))
 (segment (start 30 46.27) (end 30 48.525) (width 0.25) (layer "F.Cu") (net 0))
 (segment (start 26.19 45) (end 26.19 47.115) (width 0.25) (layer "F.Cu") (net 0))
 (segment (start 44 46.27) (end 44 48.525) (width 0.25) (layer "F.Cu") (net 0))
 (segment (start 40.19 45) (end 40.19 47.115) (width 0.25) (layer "F.Cu") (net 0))
 (segment (start 45.27 45) (end 44 46.27) (width 0.25) (layer "F.Cu") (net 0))
 (segment (start 42.73 45) (end 42.73 48.455) (width 0.25) (layer "F.Cu") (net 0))
 (segment (start 33.81 47.115) (end 32.4 48.525) (width 0.25) (layer "F.Cu") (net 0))
 (segment (start 33.81 45) (end 33.81 47.115) (width 0.25) (layer "F.Cu") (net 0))
 (segment (start 31.27 45) (end 30 46.27) (width 0.25) (layer "F.Cu") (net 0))
 (segment (start 28.73 48.455) (end 28.8 48.525) (width 0.25) (layer "F.Cu") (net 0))
 (segment (start 28.73 45) (end 28.73 48.455) (width 0.25) (layer "F.Cu") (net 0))
 (segment (start 47.81 47.115) (end 46.4 48.525) (width 0.25) (layer "F.Cu") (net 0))
 (segment (start 47.81 45) (end 47.81 47.115) (width 0.25) (layer "F.Cu") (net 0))
 (segment (start 26.19 47.115) (end 27.6 48.525) (width 0.25) (layer "F.Cu") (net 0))
 (segment (start 56.73 48.455) (end 56.8 48.525) (width 0.25) (layer "F.Cu") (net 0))
 (segment (start 54.19 47.115) (end 55.6 48.525) (width 0.25) (layer "F.Cu") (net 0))
 (segment (start 58 46.27) (end 58 48.525) (width 0.25) (layer "F.Cu") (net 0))
 (segment (start 54.19 45) (end 54.19 47.115) (width 0.25) (layer "F.Cu") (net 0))
 (segment (start 61.81 45) (end 61.81 47.115) (width 0.25) (layer "F.Cu") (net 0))
 (segment (start 59.27 45) (end 58 46.27) (width 0.25) (layer "F.Cu") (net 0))
 (segment (start 61.81 47.115) (end 60.4 48.525) (width 0.25) (layer "F.Cu") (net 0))
 (segment (start 56.73 45) (end 56.73 48.455) (width 0.25) (layer "F.Cu") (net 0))
 (segment (start 45.27 25) (end 44 26.27) (width 0.25) (layer "F.Cu") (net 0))
 (segment (start 40.19 25) (end 40.19 27.115) (width 0.25) (layer "F.Cu") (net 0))
 (segment (start 40.19 27.115) (end 41.6 28.525) (width 0.25) (layer "F.Cu") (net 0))
 (segment (start 47.81 25) (end 47.81 27.115) (width 0.25) (layer "F.Cu") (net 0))
 (segment (start 47.81 27.115) (end 46.4 28.525) (width 0.25) (layer "F.Cu") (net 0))
 (segment (start 42.73 28.455) (end 42.8 28.525) (width 0.25) (layer "F.Cu") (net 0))
 (segment (start 44 26.27) (end 44 28.525) (width 0.25) (layer "F.Cu") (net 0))
 (segment (start 42.73 25) (end 42.73 28.455) (width 0.25) (layer "F.Cu") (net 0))
 (segment (start 26.19 27.115) (end 27.6 28.525) (width 0.25) (layer "F.Cu") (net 1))
 (segment (start 26.19 25) (end 26.19 27.115) (width 0.25) (layer "F.Cu") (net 1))
 (segment (start 33.81 27.115) (end 32.4 28.525) (width 0.25) (layer "F.Cu") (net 5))
 (segment (start 33.81 25) (end 33.81 27.115) (width 0.25) (layer "F.Cu") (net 5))
 (segment (start 30 26.27) (end 30 28.525) (width 0.25) (layer "F.Cu") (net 3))
 (segment (start 31.27 25) (end 30 26.27) (width 0.25) (layer "F.Cu") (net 3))
 (segment (start 28.73 28.455) (end 28.8 28.525) (width 0.25) (layer "F.Cu") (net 2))
 (segment (start 28.73 25) (end 28.73 28.455) (width 0.25) (layer "F.Cu") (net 2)))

